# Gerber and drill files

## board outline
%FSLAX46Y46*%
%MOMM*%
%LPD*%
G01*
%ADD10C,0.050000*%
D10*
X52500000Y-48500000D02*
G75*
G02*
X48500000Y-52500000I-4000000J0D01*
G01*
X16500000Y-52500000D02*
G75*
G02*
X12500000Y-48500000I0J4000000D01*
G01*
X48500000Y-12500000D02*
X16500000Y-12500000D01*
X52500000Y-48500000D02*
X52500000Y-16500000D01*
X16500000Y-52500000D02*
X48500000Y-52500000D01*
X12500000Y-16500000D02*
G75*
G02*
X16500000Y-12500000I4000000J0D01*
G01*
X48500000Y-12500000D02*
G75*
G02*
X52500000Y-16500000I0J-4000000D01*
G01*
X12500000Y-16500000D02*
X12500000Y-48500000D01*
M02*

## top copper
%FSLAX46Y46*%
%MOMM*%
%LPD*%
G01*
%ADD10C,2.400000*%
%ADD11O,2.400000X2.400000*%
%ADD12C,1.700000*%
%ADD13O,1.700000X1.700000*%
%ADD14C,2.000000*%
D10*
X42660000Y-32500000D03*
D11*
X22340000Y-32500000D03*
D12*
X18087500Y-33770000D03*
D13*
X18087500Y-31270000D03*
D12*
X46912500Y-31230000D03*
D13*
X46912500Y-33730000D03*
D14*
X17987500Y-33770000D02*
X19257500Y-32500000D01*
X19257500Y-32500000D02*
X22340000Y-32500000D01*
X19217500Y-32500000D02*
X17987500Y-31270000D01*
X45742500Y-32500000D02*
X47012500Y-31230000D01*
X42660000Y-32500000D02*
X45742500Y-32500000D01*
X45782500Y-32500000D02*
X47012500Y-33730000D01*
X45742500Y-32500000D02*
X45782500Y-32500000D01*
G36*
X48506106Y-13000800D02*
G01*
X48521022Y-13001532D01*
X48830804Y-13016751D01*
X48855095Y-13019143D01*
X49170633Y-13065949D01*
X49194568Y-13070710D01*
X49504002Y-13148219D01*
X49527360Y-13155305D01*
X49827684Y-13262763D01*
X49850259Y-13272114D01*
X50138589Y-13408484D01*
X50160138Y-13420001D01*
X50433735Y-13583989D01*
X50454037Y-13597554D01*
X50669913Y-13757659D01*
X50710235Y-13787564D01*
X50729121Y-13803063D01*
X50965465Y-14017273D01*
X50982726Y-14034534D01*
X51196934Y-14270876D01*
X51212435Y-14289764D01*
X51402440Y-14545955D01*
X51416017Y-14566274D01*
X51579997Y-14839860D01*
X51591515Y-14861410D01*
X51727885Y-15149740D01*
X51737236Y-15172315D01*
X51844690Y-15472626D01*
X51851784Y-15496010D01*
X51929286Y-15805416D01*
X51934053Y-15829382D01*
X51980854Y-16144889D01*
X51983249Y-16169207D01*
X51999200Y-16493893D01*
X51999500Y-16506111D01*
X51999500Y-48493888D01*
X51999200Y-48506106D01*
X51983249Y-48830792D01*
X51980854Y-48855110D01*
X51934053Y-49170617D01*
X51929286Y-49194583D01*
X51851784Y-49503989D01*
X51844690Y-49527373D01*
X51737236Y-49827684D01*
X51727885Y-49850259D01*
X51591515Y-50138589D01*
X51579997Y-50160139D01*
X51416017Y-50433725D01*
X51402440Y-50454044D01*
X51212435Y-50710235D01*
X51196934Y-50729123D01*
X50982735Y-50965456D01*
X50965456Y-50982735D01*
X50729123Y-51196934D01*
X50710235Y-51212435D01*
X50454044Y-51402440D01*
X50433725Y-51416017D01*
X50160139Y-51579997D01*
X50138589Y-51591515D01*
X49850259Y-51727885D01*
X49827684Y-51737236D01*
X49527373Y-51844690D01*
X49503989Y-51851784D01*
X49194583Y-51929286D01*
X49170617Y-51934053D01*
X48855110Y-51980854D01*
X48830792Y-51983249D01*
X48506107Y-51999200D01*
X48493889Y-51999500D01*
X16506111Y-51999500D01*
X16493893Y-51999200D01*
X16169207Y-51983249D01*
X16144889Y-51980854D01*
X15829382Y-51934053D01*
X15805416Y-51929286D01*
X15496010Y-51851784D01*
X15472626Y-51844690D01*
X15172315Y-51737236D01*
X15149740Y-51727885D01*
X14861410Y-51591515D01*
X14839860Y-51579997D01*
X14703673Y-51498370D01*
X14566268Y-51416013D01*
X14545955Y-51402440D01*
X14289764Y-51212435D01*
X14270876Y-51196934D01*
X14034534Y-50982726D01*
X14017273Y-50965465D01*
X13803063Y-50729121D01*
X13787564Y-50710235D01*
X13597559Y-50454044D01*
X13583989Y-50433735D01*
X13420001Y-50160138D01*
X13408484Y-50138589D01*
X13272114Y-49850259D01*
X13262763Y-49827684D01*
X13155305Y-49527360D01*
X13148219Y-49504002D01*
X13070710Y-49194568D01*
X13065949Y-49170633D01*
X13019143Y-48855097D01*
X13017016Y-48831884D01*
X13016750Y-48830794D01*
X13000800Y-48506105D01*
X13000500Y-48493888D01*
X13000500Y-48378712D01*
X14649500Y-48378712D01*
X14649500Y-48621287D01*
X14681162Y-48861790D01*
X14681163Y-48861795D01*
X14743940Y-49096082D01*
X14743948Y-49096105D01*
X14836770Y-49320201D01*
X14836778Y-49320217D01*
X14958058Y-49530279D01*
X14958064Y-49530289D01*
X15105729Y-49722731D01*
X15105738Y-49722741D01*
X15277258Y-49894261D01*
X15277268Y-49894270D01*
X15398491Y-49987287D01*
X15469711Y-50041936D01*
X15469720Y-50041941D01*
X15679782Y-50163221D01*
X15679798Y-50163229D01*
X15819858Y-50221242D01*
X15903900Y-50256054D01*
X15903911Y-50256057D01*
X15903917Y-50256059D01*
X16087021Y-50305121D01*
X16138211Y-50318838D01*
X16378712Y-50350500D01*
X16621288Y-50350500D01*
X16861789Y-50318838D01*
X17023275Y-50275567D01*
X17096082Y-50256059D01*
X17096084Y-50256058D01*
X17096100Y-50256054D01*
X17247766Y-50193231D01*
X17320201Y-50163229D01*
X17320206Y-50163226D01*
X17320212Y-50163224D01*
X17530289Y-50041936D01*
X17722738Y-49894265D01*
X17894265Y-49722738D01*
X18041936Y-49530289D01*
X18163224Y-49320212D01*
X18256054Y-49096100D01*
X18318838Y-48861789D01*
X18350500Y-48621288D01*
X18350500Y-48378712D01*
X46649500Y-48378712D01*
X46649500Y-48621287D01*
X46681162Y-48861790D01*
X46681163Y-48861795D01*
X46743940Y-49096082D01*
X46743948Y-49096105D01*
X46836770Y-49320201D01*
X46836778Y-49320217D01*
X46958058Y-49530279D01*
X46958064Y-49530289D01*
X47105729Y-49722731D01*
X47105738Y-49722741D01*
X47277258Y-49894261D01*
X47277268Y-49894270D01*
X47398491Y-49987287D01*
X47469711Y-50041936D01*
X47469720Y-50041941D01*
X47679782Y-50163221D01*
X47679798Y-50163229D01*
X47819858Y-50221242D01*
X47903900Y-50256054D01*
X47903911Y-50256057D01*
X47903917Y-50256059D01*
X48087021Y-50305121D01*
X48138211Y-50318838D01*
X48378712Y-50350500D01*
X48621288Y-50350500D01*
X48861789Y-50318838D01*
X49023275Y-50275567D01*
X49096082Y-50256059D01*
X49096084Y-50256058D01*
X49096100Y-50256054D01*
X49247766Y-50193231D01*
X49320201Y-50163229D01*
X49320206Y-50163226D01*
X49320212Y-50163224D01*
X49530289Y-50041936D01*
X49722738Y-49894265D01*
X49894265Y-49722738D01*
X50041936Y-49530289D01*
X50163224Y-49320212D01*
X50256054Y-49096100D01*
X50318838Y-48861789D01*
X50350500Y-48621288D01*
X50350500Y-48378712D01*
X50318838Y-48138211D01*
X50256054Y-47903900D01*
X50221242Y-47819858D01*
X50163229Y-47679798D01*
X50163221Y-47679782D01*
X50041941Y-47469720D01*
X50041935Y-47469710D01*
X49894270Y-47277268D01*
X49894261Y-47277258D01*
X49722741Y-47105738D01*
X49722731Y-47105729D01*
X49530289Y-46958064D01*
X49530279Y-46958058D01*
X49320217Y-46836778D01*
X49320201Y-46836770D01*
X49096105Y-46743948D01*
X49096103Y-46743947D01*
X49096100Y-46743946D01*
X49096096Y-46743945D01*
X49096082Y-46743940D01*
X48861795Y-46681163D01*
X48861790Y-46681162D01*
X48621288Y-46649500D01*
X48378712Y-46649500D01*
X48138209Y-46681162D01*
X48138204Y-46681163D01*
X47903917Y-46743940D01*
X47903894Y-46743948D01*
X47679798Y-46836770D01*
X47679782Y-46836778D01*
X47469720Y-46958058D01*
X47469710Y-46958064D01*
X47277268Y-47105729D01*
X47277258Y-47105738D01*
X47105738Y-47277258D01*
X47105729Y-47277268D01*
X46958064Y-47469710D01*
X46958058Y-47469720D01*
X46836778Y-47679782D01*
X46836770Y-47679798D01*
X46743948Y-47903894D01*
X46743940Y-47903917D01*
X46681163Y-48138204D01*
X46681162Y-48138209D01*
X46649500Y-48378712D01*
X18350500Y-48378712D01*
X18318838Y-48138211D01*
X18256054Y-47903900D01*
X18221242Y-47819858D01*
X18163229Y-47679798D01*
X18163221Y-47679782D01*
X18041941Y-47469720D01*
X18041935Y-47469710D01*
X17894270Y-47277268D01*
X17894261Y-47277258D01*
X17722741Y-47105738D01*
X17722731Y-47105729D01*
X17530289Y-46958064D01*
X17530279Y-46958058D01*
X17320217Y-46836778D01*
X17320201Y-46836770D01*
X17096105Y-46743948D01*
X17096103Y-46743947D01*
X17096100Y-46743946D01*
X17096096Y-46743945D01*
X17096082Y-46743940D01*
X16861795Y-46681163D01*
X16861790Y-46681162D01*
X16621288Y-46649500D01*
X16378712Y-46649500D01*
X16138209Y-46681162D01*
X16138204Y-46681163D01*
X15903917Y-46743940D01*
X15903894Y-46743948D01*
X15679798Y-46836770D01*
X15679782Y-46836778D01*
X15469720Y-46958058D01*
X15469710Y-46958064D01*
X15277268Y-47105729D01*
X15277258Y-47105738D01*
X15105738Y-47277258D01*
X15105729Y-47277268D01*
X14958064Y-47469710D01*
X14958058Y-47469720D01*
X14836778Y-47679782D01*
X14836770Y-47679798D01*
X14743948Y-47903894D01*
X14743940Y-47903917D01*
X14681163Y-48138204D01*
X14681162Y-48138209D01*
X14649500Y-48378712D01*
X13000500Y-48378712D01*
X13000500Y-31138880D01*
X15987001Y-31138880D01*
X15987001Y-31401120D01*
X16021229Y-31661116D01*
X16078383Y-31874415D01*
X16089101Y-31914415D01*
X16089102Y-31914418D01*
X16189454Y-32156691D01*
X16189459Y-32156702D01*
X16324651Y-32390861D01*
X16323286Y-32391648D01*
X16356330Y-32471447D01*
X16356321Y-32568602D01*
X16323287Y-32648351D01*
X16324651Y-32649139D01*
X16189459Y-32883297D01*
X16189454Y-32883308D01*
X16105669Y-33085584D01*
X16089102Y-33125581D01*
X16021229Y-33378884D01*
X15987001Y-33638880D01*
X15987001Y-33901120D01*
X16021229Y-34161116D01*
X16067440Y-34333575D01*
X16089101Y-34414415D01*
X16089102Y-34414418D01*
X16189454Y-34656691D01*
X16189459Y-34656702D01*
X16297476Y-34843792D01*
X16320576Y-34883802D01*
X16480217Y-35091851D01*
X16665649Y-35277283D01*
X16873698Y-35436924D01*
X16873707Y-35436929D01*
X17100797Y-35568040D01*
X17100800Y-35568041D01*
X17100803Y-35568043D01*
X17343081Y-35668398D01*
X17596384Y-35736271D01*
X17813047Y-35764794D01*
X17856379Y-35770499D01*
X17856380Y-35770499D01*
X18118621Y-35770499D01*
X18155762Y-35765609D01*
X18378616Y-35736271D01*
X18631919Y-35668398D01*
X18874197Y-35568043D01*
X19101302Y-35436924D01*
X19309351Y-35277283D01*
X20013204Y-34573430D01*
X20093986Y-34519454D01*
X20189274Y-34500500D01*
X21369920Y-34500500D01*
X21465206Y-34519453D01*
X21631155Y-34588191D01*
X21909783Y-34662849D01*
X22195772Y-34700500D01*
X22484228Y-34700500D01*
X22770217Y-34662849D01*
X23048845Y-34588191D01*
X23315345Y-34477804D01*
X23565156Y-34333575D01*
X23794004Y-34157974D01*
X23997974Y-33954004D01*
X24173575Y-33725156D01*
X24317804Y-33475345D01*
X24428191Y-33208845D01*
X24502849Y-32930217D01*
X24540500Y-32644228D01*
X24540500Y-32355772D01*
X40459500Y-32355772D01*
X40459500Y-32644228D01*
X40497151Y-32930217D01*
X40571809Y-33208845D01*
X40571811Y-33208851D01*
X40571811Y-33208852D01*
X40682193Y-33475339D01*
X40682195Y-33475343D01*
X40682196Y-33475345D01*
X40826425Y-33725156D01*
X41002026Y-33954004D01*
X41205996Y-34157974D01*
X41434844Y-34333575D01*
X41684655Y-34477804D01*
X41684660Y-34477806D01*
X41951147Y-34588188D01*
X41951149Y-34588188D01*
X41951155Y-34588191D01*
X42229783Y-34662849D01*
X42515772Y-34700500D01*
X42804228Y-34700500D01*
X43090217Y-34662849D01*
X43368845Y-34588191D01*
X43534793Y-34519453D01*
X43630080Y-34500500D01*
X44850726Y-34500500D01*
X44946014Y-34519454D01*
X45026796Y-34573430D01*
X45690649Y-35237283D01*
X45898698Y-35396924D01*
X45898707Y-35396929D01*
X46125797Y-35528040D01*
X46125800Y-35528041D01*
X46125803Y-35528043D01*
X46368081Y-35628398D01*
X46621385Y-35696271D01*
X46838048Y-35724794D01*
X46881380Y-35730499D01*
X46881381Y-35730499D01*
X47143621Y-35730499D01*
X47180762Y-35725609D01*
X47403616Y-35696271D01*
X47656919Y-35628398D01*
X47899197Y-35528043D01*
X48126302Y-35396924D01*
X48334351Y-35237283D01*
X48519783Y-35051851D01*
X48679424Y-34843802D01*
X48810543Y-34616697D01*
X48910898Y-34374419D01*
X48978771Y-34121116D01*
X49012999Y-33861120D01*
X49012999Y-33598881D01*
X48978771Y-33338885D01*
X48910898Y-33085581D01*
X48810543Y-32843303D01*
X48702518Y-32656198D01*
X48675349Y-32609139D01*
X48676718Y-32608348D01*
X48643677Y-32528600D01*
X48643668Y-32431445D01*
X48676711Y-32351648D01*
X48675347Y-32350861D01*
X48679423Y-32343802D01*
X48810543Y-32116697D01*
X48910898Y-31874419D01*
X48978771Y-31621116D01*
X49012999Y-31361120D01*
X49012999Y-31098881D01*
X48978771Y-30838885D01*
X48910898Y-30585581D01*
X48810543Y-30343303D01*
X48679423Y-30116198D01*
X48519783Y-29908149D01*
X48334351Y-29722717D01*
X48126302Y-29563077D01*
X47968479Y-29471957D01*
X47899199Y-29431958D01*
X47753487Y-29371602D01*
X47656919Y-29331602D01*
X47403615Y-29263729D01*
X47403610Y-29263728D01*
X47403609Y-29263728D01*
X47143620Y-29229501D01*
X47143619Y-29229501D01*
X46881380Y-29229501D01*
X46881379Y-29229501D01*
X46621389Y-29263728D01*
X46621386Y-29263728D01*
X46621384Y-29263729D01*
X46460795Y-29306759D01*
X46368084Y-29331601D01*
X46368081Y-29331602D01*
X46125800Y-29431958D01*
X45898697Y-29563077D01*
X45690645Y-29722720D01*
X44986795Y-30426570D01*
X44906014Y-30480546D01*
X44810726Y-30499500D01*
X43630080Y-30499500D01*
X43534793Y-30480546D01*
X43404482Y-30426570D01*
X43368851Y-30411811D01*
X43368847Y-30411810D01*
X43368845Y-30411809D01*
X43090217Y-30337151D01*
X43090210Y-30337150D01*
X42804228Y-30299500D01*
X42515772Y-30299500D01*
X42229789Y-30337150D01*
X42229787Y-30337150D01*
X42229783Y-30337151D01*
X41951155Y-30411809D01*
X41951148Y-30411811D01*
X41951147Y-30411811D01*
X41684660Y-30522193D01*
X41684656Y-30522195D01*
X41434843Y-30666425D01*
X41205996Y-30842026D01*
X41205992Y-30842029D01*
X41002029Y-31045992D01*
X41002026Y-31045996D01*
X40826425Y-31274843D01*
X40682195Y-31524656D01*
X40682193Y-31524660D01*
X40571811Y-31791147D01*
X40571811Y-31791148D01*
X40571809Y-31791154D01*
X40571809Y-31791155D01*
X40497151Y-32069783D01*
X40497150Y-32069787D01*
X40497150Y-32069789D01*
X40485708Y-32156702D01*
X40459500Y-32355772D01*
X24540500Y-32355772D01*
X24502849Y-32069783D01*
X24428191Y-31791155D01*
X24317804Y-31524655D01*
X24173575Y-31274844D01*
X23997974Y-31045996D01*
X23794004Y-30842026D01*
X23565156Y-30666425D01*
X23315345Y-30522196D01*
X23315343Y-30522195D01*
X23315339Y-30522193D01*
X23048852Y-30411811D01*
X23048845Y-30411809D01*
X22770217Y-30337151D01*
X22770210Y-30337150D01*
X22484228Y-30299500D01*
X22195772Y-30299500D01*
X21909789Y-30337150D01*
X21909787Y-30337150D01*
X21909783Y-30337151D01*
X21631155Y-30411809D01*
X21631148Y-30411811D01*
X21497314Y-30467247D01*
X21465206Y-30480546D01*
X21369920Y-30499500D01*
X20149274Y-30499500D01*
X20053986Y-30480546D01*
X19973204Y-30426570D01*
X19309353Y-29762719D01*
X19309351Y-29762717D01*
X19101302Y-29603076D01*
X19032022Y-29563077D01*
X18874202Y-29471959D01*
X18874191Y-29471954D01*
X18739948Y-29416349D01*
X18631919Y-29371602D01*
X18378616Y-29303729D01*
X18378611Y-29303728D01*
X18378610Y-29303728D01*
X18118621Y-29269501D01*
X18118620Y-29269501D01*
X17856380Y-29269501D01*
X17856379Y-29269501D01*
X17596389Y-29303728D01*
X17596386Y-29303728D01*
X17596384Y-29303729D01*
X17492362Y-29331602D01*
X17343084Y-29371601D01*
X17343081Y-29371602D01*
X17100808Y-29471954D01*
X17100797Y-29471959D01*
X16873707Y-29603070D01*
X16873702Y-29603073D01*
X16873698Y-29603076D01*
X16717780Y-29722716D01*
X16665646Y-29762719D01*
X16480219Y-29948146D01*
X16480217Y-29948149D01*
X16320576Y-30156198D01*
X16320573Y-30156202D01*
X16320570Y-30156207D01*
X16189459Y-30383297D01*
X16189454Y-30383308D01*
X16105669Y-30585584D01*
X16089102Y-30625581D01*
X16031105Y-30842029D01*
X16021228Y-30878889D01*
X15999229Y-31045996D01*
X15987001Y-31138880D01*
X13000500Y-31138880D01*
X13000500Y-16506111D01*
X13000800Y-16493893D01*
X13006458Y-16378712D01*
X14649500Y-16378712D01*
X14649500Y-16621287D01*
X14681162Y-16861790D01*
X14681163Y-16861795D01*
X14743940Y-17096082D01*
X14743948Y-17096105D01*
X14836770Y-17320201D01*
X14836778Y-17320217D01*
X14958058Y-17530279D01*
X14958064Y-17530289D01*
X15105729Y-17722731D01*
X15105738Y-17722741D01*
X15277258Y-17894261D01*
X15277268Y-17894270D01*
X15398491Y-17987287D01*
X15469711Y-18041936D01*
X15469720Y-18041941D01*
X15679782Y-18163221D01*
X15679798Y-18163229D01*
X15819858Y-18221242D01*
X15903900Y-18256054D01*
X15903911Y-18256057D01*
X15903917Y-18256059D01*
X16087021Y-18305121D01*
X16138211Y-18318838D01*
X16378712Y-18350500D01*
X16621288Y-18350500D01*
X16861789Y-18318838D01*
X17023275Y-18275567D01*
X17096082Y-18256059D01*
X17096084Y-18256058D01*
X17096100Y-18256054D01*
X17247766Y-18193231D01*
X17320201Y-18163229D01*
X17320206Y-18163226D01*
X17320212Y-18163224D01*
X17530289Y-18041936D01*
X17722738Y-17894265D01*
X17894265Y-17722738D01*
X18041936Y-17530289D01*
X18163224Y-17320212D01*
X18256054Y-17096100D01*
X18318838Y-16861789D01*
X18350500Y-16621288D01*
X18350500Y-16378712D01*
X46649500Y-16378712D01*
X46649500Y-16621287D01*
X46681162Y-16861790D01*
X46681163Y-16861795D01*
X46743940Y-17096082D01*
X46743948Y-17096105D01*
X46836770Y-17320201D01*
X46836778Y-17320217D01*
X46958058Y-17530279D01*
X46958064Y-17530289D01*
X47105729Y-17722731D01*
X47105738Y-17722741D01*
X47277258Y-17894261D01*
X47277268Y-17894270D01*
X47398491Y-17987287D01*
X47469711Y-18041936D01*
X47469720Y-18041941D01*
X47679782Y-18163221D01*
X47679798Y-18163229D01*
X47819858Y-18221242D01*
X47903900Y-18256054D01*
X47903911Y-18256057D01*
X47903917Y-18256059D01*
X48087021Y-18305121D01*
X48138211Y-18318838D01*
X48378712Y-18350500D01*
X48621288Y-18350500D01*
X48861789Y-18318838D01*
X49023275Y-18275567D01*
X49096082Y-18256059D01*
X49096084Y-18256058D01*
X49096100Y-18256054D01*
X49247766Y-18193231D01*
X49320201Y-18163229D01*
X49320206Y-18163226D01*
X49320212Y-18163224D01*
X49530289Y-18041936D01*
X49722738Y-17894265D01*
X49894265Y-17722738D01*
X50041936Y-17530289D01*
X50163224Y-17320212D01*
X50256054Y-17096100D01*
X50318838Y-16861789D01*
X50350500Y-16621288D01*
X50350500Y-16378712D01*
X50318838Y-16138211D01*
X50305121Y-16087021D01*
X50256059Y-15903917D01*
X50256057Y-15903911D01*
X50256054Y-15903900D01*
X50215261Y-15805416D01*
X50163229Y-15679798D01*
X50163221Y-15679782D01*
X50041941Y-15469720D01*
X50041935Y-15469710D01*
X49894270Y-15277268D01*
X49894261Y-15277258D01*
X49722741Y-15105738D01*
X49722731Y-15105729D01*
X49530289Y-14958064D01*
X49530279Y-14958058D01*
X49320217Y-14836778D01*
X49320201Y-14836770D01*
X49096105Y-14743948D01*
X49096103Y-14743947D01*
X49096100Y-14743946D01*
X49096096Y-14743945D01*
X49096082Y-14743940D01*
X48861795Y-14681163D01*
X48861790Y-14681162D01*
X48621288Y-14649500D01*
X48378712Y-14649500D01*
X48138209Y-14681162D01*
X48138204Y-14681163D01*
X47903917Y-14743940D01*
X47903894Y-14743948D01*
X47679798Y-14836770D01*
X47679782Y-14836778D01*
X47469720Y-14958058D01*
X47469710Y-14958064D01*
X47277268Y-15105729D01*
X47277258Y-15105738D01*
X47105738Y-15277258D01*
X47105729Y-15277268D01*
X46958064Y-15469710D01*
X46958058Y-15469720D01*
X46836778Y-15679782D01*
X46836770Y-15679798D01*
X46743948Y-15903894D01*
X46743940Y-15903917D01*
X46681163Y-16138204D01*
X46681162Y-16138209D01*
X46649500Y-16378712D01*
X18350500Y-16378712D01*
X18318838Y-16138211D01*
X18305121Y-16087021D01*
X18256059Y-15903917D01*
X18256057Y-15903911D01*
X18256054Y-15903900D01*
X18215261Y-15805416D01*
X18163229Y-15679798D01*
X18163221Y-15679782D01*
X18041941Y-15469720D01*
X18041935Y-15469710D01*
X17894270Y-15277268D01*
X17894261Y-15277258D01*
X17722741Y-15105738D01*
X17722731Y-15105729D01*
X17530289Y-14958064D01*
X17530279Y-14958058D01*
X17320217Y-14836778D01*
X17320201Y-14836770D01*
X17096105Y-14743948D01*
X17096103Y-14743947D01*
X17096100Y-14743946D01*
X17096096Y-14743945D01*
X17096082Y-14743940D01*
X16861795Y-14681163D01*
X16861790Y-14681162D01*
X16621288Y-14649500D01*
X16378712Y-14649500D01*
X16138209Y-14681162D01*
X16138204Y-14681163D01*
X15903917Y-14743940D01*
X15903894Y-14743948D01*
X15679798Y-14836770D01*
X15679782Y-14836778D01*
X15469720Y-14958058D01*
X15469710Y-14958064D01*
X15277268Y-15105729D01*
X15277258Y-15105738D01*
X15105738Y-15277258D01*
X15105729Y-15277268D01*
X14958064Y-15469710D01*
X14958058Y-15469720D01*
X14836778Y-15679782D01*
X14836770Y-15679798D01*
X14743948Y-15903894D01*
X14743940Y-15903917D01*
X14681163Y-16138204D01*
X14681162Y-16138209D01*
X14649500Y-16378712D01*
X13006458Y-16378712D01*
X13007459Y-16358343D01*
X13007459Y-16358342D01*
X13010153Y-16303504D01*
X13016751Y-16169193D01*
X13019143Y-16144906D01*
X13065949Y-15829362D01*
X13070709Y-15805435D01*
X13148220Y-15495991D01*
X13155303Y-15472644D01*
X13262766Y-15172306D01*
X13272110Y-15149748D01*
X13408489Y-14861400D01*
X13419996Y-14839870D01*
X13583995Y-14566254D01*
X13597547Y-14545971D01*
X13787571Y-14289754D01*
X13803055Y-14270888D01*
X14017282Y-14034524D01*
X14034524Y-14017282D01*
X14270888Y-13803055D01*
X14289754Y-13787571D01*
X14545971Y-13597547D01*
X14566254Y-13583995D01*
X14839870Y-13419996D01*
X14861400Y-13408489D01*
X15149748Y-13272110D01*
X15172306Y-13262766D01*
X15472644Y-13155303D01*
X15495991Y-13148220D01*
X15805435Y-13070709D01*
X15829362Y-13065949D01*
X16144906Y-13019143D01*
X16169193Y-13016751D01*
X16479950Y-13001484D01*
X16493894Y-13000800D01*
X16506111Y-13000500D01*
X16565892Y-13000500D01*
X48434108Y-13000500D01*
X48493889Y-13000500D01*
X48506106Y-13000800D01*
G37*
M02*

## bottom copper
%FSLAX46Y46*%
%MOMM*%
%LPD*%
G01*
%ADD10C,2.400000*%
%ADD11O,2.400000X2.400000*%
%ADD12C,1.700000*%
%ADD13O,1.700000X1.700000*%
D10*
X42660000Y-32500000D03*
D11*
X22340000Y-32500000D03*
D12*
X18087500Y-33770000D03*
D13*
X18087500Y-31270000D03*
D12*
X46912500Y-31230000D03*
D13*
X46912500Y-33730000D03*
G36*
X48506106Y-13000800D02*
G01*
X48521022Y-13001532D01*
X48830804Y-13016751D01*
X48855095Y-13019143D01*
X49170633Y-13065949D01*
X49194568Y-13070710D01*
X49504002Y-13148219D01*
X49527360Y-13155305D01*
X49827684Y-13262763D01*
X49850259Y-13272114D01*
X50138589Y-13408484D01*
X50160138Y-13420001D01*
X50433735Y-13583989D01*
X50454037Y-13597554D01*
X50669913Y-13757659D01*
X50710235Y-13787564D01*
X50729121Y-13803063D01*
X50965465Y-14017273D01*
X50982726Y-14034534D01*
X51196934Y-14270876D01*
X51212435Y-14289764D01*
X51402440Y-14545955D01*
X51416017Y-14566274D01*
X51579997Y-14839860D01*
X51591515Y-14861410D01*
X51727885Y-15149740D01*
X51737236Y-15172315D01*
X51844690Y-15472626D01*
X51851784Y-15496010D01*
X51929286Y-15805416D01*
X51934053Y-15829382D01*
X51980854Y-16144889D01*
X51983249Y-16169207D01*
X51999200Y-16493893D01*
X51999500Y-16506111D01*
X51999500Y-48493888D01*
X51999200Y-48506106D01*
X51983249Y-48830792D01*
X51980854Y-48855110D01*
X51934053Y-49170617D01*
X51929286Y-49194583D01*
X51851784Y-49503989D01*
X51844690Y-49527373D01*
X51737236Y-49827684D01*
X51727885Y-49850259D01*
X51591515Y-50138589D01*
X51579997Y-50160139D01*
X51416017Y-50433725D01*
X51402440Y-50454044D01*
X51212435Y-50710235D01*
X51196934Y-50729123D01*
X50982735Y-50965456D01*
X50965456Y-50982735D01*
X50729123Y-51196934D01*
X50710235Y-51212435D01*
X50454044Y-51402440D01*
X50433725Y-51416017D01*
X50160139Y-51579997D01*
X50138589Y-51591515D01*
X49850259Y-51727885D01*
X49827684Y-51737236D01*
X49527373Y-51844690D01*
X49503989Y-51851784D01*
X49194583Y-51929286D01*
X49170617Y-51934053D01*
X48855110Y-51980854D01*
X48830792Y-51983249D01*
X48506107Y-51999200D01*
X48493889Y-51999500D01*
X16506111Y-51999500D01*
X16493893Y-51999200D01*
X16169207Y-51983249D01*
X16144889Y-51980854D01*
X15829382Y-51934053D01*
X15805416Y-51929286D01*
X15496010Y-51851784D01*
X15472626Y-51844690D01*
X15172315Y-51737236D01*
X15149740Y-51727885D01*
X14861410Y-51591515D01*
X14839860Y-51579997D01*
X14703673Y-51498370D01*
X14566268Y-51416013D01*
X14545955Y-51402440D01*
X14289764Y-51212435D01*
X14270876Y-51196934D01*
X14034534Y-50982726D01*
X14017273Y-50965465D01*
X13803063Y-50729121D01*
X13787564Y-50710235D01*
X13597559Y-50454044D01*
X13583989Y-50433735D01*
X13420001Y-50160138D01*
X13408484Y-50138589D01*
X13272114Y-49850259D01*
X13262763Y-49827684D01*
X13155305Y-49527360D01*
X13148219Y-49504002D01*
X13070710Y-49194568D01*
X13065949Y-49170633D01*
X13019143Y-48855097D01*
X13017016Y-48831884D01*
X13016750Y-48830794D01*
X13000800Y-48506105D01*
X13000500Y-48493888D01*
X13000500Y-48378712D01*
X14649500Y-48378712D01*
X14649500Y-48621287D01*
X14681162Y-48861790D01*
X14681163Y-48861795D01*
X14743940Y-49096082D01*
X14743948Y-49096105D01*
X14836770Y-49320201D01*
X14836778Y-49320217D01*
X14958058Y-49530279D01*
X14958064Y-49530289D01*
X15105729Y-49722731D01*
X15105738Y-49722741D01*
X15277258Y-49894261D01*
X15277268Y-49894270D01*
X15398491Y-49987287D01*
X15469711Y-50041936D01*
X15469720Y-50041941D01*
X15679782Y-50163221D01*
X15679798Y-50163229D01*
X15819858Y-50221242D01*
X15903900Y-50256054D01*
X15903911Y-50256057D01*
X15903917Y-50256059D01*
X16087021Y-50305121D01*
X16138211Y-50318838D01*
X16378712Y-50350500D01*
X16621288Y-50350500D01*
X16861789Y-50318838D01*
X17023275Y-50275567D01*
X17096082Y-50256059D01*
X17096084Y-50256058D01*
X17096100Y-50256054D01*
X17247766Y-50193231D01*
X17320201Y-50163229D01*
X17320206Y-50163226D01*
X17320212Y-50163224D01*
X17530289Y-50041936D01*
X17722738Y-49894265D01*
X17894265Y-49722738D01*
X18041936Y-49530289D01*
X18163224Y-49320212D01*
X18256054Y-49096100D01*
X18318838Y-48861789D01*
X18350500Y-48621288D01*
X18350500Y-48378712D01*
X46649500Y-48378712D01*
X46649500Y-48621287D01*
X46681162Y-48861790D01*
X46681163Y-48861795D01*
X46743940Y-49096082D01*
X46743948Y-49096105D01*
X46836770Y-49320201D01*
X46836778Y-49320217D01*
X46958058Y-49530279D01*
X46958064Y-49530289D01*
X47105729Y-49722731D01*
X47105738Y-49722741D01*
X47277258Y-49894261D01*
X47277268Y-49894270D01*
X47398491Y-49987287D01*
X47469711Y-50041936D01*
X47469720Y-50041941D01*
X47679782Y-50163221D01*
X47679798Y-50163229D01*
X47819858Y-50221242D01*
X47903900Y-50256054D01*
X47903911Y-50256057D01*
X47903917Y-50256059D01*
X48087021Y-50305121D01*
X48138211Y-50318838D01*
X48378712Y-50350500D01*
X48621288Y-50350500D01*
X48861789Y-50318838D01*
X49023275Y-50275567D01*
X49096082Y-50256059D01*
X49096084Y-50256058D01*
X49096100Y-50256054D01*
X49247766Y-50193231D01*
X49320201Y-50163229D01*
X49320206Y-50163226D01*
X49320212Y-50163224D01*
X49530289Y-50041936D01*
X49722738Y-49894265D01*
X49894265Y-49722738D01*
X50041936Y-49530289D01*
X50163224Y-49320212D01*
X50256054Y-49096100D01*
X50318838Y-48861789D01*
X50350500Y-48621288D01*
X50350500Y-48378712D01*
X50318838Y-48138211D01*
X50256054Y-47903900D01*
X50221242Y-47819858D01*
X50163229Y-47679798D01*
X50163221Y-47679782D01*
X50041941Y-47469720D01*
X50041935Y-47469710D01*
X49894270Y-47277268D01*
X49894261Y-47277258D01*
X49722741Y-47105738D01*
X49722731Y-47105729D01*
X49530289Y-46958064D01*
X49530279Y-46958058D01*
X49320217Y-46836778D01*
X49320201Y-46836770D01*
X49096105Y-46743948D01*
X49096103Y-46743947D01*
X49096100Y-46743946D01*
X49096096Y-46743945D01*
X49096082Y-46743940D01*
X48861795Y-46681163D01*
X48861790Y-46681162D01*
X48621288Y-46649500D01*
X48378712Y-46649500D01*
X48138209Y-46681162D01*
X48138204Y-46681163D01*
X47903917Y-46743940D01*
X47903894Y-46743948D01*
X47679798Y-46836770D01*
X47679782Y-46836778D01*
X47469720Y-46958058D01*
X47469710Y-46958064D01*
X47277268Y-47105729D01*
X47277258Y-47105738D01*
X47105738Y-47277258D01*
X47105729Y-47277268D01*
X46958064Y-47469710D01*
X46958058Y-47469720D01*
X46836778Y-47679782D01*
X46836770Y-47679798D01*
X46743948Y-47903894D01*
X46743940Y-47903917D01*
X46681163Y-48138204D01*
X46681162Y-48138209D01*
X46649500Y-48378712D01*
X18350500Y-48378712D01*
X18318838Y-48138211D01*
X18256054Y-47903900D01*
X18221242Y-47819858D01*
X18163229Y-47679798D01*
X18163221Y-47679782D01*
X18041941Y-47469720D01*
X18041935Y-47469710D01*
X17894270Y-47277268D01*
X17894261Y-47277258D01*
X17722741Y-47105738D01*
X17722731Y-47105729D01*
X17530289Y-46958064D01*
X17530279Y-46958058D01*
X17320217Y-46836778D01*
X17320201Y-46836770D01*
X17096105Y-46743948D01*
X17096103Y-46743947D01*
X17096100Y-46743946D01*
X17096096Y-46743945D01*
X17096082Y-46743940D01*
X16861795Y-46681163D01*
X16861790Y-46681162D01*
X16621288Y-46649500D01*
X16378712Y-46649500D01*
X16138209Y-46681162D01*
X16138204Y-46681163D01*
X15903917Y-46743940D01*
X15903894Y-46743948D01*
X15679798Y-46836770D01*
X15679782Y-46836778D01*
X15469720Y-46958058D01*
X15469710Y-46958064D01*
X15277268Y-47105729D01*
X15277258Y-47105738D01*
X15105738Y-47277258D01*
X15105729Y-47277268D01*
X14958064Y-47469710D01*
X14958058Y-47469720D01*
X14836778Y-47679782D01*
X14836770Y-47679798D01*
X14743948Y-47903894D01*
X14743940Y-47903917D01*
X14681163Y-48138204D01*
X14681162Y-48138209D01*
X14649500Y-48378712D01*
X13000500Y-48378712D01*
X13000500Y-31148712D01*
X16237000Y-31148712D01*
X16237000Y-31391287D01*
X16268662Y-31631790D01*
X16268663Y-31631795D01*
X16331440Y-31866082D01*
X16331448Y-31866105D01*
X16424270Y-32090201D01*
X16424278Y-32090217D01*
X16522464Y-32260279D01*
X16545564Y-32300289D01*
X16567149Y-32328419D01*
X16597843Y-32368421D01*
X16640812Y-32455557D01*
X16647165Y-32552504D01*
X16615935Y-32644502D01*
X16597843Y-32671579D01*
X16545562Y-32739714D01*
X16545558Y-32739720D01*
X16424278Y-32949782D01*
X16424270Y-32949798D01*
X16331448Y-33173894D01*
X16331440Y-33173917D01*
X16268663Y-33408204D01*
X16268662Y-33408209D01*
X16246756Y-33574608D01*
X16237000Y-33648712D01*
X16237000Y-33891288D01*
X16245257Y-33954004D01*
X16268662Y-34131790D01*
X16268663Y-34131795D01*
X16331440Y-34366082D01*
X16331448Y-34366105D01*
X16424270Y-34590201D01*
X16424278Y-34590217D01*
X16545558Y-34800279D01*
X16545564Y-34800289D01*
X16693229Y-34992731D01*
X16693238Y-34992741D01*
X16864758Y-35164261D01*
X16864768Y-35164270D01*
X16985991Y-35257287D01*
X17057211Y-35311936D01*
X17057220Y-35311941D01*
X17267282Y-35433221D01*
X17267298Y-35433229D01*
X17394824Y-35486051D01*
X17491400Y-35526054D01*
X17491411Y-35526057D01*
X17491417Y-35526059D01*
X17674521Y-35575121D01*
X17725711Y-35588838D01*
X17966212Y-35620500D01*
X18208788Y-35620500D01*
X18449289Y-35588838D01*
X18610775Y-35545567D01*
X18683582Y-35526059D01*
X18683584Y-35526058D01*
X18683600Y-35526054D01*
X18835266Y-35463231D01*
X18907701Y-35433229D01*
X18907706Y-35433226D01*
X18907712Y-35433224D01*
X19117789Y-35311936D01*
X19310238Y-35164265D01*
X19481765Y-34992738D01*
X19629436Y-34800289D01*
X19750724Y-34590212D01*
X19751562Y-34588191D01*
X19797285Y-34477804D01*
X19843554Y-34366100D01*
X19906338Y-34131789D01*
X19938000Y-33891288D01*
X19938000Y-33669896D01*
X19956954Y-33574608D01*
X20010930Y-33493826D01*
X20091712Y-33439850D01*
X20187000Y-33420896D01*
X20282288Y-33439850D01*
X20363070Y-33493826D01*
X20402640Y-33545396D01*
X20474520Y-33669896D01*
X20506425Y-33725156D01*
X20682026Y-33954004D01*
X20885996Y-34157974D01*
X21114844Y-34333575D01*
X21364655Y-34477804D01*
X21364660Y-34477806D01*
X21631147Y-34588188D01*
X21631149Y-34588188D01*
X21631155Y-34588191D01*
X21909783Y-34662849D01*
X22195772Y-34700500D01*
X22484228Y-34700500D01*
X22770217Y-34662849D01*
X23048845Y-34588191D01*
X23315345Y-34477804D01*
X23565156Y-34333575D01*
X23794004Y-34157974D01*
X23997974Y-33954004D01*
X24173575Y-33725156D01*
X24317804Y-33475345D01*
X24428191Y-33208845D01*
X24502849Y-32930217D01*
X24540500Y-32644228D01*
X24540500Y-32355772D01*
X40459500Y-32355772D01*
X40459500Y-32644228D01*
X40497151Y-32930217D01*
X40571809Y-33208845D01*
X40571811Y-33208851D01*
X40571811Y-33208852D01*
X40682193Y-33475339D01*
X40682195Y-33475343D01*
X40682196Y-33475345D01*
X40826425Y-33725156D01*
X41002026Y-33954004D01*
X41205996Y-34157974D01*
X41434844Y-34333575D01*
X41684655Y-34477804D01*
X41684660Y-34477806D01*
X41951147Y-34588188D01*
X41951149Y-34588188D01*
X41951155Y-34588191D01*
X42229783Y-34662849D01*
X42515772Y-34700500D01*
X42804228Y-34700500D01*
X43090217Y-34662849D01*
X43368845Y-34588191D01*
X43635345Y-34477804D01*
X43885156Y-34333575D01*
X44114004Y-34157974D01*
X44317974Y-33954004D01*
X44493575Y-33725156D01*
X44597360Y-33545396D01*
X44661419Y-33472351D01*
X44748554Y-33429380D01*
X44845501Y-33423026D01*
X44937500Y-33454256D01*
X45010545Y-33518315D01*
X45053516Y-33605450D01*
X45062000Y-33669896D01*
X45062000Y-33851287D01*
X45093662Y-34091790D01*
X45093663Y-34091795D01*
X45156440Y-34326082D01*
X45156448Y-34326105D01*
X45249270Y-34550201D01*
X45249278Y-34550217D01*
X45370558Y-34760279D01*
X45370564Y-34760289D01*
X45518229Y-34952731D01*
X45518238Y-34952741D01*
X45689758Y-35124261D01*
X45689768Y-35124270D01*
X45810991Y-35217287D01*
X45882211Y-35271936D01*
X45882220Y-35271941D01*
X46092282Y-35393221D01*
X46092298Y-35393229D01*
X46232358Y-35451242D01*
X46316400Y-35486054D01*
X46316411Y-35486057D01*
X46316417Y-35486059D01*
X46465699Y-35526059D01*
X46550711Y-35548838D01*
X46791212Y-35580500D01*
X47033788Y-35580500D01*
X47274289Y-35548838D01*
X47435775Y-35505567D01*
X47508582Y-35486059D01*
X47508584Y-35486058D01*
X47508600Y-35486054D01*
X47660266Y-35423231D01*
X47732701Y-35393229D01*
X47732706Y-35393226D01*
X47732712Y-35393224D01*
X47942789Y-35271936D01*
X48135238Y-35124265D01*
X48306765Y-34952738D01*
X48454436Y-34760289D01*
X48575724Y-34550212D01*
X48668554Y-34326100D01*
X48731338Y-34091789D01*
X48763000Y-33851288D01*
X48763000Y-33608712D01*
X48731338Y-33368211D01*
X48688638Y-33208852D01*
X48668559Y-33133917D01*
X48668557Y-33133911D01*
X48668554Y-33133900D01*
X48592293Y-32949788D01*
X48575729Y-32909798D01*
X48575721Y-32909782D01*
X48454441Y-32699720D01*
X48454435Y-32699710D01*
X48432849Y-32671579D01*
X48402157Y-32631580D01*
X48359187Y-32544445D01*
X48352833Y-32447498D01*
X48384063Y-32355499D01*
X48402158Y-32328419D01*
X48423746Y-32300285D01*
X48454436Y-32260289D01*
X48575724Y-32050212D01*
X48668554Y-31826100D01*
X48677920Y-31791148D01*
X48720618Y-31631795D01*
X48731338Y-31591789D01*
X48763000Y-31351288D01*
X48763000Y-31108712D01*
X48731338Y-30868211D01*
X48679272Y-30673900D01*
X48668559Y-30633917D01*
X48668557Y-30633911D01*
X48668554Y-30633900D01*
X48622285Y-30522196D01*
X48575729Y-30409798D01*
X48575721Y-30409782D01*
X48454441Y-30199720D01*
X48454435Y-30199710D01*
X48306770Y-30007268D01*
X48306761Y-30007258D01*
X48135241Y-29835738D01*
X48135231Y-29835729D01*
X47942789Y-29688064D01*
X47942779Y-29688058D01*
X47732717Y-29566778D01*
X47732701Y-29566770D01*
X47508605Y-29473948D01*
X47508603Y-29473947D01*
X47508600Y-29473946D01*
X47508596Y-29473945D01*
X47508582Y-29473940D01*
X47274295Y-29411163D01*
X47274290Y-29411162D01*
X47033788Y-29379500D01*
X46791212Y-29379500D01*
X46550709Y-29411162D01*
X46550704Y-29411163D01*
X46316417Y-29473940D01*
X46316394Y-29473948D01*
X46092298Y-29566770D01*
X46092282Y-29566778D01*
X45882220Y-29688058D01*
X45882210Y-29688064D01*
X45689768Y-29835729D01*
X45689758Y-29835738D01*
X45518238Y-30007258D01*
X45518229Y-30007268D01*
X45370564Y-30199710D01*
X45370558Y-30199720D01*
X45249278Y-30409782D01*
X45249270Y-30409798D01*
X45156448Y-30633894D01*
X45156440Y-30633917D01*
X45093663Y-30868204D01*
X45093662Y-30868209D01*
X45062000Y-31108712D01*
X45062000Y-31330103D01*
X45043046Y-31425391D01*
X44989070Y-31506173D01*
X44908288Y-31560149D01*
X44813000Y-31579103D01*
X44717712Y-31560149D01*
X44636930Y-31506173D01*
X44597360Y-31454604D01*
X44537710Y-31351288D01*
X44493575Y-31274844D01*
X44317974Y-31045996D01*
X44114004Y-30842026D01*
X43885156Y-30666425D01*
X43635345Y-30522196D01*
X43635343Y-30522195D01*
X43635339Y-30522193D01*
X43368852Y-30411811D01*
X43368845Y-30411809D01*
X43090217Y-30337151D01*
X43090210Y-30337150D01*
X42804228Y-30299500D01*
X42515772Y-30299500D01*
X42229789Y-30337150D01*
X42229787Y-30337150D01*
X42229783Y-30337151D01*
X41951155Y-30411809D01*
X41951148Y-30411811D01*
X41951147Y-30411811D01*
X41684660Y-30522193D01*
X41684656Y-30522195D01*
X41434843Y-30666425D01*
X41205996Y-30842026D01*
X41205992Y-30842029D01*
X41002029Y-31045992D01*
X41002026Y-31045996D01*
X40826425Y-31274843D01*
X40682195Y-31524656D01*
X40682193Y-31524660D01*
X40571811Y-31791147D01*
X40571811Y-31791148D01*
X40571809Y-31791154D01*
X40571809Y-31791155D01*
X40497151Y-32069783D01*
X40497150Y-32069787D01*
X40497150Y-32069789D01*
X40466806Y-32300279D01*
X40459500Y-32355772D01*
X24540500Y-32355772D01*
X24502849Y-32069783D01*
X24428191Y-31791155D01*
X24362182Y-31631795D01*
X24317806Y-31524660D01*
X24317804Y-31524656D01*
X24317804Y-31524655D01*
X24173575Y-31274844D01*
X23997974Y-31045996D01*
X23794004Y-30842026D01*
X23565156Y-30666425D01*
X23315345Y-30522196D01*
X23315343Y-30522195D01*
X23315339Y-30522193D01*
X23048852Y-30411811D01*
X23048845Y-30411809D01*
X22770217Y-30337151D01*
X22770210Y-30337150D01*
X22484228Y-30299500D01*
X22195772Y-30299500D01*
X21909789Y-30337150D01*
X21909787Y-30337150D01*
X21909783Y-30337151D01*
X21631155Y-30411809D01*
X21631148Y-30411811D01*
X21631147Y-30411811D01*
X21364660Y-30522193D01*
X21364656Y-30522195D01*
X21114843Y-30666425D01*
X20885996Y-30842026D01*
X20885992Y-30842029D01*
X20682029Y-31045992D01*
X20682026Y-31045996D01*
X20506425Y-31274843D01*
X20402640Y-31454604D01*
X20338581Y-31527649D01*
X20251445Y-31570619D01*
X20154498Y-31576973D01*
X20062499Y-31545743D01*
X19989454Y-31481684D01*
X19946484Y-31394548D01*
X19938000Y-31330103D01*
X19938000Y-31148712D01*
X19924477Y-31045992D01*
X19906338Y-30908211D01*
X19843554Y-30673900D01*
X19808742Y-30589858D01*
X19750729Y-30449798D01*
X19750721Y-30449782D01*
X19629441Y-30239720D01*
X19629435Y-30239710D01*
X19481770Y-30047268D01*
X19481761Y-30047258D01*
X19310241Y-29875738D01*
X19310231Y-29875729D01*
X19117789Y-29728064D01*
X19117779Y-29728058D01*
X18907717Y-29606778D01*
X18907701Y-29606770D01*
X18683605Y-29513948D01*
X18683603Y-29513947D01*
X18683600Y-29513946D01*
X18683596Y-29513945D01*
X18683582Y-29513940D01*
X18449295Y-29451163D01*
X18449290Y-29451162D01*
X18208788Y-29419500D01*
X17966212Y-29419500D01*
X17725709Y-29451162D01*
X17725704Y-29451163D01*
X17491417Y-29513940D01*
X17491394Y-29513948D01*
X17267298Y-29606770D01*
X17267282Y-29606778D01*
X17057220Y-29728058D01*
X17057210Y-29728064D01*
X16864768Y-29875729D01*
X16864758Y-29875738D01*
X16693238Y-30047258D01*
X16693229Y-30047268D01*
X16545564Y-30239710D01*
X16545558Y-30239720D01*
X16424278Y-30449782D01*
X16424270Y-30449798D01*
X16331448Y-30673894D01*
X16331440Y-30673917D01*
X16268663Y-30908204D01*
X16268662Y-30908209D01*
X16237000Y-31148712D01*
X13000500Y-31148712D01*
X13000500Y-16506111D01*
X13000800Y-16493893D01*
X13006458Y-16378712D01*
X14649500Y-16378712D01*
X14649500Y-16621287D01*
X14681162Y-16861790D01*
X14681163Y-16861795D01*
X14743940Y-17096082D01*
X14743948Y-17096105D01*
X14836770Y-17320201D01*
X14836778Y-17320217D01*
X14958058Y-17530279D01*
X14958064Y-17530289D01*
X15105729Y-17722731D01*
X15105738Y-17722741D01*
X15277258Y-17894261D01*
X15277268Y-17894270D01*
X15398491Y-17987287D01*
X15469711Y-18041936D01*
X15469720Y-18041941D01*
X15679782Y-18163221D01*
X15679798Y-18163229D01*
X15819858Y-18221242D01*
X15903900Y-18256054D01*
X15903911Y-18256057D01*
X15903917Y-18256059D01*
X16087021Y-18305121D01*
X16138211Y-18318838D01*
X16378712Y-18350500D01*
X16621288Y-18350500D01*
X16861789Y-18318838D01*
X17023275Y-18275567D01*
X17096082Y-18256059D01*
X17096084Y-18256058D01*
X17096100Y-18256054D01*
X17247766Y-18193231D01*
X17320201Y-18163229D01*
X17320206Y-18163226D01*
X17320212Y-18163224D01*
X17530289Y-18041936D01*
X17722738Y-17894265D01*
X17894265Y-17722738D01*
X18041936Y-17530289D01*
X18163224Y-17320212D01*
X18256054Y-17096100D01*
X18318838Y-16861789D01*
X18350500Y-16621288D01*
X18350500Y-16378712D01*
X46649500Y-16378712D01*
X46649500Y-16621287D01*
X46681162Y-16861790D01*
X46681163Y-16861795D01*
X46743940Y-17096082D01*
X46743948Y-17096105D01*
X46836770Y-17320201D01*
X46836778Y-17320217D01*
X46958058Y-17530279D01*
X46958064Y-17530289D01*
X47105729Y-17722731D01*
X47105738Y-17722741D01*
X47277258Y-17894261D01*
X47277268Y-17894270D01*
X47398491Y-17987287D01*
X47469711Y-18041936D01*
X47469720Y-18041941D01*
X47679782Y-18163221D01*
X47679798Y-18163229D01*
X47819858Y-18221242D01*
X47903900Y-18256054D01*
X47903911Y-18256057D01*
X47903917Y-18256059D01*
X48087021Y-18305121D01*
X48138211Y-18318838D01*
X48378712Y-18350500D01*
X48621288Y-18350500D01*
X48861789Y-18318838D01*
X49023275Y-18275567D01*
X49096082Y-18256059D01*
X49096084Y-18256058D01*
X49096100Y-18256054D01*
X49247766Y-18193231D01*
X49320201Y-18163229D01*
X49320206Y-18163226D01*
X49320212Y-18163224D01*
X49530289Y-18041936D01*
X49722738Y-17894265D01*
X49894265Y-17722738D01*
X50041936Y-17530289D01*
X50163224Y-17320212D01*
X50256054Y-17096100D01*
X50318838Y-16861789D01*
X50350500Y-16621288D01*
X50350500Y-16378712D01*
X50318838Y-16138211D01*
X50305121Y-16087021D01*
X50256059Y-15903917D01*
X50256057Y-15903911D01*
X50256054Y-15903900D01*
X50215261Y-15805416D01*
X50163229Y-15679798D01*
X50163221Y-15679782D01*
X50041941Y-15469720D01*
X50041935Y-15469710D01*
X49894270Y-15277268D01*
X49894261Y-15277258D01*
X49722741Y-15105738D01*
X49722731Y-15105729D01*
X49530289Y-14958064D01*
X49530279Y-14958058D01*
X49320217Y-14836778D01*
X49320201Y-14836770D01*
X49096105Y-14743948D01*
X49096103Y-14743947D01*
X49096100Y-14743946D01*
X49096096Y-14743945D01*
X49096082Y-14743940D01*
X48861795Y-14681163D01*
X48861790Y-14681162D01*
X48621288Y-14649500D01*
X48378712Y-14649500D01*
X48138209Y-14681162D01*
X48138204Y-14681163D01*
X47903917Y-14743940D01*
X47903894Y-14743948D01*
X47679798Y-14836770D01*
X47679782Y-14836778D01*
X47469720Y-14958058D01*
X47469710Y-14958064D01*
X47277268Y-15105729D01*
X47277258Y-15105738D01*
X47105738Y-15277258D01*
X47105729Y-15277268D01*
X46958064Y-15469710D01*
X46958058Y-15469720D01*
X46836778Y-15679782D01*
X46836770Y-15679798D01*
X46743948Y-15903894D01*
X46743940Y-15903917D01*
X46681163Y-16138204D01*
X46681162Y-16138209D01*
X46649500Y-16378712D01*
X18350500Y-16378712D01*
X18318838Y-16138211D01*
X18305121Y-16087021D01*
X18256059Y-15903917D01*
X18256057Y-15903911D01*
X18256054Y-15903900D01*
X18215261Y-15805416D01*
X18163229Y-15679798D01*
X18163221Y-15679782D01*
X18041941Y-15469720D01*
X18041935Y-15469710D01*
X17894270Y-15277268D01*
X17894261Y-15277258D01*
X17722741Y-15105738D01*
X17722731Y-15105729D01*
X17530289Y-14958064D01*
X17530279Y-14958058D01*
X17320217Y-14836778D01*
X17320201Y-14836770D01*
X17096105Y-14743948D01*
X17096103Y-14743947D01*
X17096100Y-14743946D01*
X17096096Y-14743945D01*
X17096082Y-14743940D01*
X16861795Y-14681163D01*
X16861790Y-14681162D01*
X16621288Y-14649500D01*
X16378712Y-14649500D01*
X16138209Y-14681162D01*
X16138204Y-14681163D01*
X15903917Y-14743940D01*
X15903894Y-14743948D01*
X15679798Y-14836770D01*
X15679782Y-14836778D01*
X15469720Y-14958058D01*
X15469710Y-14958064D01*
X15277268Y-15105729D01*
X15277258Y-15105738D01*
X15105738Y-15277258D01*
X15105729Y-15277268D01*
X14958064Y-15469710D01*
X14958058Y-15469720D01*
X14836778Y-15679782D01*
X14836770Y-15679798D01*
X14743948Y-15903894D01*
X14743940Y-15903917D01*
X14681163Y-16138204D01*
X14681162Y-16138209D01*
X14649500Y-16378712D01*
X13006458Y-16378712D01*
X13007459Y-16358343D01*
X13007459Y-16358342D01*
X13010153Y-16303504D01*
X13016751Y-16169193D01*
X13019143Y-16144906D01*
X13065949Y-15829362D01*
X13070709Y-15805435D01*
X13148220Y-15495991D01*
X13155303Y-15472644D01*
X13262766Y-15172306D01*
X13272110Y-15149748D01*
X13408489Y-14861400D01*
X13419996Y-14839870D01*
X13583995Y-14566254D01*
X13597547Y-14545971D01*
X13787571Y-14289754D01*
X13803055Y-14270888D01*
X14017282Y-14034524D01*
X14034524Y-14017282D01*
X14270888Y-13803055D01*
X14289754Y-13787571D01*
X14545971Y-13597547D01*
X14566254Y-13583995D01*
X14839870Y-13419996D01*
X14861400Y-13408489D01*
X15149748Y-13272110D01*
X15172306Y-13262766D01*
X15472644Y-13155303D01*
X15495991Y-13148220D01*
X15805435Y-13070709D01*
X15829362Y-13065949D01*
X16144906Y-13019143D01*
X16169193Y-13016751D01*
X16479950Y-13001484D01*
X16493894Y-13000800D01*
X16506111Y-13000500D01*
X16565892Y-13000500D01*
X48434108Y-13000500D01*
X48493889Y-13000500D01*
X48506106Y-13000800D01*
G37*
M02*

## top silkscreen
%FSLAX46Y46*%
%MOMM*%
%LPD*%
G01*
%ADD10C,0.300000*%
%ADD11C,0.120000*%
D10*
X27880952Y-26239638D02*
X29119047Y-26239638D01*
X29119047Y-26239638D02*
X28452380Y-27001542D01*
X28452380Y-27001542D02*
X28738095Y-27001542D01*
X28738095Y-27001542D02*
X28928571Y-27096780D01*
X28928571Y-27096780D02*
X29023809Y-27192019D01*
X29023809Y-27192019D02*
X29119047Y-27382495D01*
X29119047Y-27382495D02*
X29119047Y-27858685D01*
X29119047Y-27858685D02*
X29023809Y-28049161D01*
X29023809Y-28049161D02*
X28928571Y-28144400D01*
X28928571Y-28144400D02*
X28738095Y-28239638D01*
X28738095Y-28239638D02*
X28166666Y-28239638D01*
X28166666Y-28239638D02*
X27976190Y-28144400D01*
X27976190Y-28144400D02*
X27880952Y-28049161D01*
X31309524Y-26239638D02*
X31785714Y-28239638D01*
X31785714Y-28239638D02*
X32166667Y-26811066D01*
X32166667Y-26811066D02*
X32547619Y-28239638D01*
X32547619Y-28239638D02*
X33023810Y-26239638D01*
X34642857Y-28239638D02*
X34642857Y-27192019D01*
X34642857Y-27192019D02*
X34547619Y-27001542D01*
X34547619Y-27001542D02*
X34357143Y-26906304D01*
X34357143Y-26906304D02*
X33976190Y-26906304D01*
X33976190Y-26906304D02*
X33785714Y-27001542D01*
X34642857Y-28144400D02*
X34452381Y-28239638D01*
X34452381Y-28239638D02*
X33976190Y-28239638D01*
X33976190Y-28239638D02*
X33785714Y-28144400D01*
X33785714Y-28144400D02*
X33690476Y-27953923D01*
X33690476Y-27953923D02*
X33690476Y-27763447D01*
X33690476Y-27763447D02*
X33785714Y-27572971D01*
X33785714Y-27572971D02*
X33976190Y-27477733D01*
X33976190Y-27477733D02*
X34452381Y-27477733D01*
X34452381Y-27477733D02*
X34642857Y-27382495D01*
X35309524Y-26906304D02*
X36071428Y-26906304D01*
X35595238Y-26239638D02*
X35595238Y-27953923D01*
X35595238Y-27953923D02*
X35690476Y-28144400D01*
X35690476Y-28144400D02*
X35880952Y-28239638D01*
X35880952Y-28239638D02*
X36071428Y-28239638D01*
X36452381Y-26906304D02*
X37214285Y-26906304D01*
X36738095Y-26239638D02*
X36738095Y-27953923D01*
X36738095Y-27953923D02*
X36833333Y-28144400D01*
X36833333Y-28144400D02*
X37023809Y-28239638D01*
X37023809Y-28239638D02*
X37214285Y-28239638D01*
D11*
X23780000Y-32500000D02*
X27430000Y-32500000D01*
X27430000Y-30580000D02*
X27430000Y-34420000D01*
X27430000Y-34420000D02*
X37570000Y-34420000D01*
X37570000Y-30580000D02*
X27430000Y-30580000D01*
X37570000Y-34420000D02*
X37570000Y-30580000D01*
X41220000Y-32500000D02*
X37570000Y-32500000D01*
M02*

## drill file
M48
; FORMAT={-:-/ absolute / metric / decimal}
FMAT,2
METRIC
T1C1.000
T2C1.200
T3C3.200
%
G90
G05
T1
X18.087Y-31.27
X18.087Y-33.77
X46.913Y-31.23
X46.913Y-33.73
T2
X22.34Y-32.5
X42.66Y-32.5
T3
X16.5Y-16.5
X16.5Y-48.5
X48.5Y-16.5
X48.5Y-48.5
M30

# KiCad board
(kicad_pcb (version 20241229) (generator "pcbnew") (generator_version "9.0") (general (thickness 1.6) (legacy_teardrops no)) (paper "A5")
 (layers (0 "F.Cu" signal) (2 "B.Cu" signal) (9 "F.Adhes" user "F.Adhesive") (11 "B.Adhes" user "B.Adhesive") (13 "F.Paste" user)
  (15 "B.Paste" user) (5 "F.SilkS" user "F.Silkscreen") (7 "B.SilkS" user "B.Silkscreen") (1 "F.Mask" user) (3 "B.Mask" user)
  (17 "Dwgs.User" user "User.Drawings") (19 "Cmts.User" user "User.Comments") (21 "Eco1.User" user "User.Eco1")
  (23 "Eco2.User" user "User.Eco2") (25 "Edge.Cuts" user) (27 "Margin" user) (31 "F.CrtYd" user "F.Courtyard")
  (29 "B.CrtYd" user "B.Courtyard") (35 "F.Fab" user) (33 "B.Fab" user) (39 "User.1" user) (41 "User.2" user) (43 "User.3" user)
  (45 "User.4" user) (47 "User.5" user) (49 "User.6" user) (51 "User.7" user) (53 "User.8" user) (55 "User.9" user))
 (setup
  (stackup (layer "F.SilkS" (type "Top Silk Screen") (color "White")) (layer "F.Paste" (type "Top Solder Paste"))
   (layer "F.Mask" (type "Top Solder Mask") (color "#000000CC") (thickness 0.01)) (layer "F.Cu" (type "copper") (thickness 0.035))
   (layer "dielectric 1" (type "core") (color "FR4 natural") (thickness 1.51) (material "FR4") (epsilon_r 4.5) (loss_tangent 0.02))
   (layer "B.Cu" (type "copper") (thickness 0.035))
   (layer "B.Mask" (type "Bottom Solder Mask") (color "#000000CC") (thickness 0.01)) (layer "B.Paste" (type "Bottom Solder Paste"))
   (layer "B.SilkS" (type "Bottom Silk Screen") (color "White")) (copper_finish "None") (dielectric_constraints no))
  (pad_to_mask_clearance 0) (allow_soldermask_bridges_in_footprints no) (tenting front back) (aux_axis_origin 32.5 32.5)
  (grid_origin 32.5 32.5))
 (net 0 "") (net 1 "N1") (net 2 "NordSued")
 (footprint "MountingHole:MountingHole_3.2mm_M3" (layer "F.Cu") (at 48.5 48.5 -90)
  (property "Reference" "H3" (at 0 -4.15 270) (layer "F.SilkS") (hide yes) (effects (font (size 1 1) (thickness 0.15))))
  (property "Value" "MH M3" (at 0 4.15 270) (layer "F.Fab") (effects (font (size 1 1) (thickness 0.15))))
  (pad "" np_thru_hole circle (at 0 0 270) (size 3.2 3.2) (drill 3.2) (layers "*.Cu" "*.Mask")))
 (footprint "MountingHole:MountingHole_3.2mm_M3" (layer "F.Cu") (at 48.5 16.5 -90)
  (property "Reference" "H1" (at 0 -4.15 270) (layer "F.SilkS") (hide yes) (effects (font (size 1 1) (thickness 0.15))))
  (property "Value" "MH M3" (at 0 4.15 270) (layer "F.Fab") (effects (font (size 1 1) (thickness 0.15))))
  (pad "" np_thru_hole circle (at 0 0 270) (size 3.2 3.2) (drill 3.2) (layers "*.Cu" "*.Mask")))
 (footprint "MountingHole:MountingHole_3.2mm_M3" (layer "F.Cu") (at 16.5 48.5 -90)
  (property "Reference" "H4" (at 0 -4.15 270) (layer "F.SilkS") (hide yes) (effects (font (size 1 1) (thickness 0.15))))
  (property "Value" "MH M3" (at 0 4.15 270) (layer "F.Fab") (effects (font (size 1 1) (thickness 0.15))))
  (pad "" np_thru_hole circle (at 0 0 270) (size 3.2 3.2) (drill 3.2) (layers "*.Cu" "*.Mask")))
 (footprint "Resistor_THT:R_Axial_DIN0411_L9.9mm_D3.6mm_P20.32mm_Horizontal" (layer "F.Cu") (at 42.66 32.5 180)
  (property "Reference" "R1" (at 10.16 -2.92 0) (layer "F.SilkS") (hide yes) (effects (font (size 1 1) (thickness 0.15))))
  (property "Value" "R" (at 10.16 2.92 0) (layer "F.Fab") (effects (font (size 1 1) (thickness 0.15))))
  (fp_line (start 18.88 0) (end 15.23 0) (stroke (width 0.12) (type solid)) (layer "F.SilkS"))
  (fp_line (start 15.23 1.92) (end 15.23 -1.92) (stroke (width 0.12) (type solid)) (layer "F.SilkS"))
  (fp_line (start 15.23 -1.92) (end 5.09 -1.92) (stroke (width 0.12) (type solid)) (layer "F.SilkS"))
  (fp_line (start 5.09 1.92) (end 15.23 1.92) (stroke (width 0.12) (type solid)) (layer "F.SilkS"))
  (fp_line (start 5.09 -1.92) (end 5.09 1.92) (stroke (width 0.12) (type solid)) (layer "F.SilkS"))
  (fp_line (start 1.44 0) (end 5.09 0) (stroke (width 0.12) (type solid)) (layer "F.SilkS"))
  (pad "1" thru_hole circle (at 0 0 180) (size 2.4 2.4) (drill 1.2) (layers "*.Cu" "*.Mask") (remove_unused_layers no) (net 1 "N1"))
  (pad "2" thru_hole oval (at 20.32 0 180) (size 2.4 2.4) (drill 1.2) (layers "*.Cu" "*.Mask") (remove_unused_layers no) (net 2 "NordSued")))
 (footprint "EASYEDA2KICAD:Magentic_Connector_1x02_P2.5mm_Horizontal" (layer "F.Cu") (at 17.9875 32.5 180)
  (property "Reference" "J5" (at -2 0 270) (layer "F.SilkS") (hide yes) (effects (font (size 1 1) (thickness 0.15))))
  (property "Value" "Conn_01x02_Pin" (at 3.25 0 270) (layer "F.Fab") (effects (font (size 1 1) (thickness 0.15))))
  (pad "1" thru_hole circle (at -0.1 -1.27 180) (size 1.7 1.7) (drill 1) (layers "*.Cu" "*.Mask") (remove_unused_layers no)
   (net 2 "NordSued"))
  (pad "2" thru_hole oval (at -0.1 1.23 180) (size 1.7 1.7) (drill 1) (layers "*.Cu" "*.Mask") (remove_unused_layers no) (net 2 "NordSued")))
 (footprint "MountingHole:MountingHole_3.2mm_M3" (layer "F.Cu") (at 16.5 16.5 -90)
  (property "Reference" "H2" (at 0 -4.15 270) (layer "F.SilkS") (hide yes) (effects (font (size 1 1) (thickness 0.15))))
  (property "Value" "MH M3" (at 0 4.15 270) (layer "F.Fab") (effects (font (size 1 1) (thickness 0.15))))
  (pad "" np_thru_hole circle (at 0 0 270) (size 3.2 3.2) (drill 3.2) (layers "*.Cu" "*.Mask")))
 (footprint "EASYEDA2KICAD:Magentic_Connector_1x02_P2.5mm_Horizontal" (layer "F.Cu") (at 47.0125 32.5)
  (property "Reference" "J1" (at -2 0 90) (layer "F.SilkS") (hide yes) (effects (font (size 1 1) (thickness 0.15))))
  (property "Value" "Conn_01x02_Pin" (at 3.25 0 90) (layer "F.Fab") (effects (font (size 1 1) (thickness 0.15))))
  (pad "1" thru_hole circle (at -0.1 -1.27) (size 1.7 1.7) (drill 1) (layers "*.Cu" "*.Mask") (remove_unused_layers no) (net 1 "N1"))
  (pad "2" thru_hole oval (at -0.1 1.23) (size 1.7 1.7) (drill 1) (layers "*.Cu" "*.Mask") (remove_unused_layers no) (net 1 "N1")))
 (gr_arc (start 52.5 48.5) (mid 51.328427 51.328427) (end 48.5 52.5) (stroke (width 0.05) (type default)) (layer "Edge.Cuts"))
 (gr_arc (start 16.5 52.5) (mid 13.671573 51.328427) (end 12.5 48.5) (stroke (width 0.05) (type default)) (layer "Edge.Cuts"))
 (gr_line (start 48.5 12.5) (end 16.5 12.5) (stroke (width 0.05) (type default)) (layer "Edge.Cuts"))
 (gr_line (start 52.5 48.5) (end 52.5 16.5) (stroke (width 0.05) (type default)) (layer "Edge.Cuts"))
 (gr_line (start 16.5 52.5) (end 48.5 52.5) (stroke (width 0.05) (type default)) (layer "Edge.Cuts"))
 (gr_arc (start 12.5 16.5) (mid 13.671573 13.671573) (end 16.5 12.5) (stroke (width 0.05) (type default)) (layer "Edge.Cuts"))
 (gr_arc (start 48.5 12.5) (mid 51.328427 13.671573) (end 52.5 16.5) (stroke (width 0.05) (type default)) (layer "Edge.Cuts"))
 (gr_line (start 12.5 16.5) (end 12.5 48.5) (stroke (width 0.05) (type default)) (layer "Edge.Cuts"))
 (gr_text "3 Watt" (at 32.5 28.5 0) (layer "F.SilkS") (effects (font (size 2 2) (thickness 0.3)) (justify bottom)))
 (segment (start 17.9875 33.77) (end 19.2575 32.5) (width 2) (layer "F.Cu") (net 2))
 (segment (start 19.2575 32.5) (end 22.34 32.5) (width 2) (layer "F.Cu") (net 2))
 (segment (start 19.2175 32.5) (end 17.9875 31.27) (width 2) (layer "F.Cu") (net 2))
 (segment (start 45.7425 32.5) (end 47.0125 31.23) (width 2) (layer "F.Cu") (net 1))
 (segment (start 42.66 32.5) (end 45.7425 32.5) (width 2) (layer "F.Cu") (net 1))
 (segment (start 45.7825 32.5) (end 47.0125 33.73) (width 2) (layer "F.Cu") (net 1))
 (segment (start 45.7425 32.5) (end 45.7825 32.5) (width 2) (layer "F.Cu") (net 1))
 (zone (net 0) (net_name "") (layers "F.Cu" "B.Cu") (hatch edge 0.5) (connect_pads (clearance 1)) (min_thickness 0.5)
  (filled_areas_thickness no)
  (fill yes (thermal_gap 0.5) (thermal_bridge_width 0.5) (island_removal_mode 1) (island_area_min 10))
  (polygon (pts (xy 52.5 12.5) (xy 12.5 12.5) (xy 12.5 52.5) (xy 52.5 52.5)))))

